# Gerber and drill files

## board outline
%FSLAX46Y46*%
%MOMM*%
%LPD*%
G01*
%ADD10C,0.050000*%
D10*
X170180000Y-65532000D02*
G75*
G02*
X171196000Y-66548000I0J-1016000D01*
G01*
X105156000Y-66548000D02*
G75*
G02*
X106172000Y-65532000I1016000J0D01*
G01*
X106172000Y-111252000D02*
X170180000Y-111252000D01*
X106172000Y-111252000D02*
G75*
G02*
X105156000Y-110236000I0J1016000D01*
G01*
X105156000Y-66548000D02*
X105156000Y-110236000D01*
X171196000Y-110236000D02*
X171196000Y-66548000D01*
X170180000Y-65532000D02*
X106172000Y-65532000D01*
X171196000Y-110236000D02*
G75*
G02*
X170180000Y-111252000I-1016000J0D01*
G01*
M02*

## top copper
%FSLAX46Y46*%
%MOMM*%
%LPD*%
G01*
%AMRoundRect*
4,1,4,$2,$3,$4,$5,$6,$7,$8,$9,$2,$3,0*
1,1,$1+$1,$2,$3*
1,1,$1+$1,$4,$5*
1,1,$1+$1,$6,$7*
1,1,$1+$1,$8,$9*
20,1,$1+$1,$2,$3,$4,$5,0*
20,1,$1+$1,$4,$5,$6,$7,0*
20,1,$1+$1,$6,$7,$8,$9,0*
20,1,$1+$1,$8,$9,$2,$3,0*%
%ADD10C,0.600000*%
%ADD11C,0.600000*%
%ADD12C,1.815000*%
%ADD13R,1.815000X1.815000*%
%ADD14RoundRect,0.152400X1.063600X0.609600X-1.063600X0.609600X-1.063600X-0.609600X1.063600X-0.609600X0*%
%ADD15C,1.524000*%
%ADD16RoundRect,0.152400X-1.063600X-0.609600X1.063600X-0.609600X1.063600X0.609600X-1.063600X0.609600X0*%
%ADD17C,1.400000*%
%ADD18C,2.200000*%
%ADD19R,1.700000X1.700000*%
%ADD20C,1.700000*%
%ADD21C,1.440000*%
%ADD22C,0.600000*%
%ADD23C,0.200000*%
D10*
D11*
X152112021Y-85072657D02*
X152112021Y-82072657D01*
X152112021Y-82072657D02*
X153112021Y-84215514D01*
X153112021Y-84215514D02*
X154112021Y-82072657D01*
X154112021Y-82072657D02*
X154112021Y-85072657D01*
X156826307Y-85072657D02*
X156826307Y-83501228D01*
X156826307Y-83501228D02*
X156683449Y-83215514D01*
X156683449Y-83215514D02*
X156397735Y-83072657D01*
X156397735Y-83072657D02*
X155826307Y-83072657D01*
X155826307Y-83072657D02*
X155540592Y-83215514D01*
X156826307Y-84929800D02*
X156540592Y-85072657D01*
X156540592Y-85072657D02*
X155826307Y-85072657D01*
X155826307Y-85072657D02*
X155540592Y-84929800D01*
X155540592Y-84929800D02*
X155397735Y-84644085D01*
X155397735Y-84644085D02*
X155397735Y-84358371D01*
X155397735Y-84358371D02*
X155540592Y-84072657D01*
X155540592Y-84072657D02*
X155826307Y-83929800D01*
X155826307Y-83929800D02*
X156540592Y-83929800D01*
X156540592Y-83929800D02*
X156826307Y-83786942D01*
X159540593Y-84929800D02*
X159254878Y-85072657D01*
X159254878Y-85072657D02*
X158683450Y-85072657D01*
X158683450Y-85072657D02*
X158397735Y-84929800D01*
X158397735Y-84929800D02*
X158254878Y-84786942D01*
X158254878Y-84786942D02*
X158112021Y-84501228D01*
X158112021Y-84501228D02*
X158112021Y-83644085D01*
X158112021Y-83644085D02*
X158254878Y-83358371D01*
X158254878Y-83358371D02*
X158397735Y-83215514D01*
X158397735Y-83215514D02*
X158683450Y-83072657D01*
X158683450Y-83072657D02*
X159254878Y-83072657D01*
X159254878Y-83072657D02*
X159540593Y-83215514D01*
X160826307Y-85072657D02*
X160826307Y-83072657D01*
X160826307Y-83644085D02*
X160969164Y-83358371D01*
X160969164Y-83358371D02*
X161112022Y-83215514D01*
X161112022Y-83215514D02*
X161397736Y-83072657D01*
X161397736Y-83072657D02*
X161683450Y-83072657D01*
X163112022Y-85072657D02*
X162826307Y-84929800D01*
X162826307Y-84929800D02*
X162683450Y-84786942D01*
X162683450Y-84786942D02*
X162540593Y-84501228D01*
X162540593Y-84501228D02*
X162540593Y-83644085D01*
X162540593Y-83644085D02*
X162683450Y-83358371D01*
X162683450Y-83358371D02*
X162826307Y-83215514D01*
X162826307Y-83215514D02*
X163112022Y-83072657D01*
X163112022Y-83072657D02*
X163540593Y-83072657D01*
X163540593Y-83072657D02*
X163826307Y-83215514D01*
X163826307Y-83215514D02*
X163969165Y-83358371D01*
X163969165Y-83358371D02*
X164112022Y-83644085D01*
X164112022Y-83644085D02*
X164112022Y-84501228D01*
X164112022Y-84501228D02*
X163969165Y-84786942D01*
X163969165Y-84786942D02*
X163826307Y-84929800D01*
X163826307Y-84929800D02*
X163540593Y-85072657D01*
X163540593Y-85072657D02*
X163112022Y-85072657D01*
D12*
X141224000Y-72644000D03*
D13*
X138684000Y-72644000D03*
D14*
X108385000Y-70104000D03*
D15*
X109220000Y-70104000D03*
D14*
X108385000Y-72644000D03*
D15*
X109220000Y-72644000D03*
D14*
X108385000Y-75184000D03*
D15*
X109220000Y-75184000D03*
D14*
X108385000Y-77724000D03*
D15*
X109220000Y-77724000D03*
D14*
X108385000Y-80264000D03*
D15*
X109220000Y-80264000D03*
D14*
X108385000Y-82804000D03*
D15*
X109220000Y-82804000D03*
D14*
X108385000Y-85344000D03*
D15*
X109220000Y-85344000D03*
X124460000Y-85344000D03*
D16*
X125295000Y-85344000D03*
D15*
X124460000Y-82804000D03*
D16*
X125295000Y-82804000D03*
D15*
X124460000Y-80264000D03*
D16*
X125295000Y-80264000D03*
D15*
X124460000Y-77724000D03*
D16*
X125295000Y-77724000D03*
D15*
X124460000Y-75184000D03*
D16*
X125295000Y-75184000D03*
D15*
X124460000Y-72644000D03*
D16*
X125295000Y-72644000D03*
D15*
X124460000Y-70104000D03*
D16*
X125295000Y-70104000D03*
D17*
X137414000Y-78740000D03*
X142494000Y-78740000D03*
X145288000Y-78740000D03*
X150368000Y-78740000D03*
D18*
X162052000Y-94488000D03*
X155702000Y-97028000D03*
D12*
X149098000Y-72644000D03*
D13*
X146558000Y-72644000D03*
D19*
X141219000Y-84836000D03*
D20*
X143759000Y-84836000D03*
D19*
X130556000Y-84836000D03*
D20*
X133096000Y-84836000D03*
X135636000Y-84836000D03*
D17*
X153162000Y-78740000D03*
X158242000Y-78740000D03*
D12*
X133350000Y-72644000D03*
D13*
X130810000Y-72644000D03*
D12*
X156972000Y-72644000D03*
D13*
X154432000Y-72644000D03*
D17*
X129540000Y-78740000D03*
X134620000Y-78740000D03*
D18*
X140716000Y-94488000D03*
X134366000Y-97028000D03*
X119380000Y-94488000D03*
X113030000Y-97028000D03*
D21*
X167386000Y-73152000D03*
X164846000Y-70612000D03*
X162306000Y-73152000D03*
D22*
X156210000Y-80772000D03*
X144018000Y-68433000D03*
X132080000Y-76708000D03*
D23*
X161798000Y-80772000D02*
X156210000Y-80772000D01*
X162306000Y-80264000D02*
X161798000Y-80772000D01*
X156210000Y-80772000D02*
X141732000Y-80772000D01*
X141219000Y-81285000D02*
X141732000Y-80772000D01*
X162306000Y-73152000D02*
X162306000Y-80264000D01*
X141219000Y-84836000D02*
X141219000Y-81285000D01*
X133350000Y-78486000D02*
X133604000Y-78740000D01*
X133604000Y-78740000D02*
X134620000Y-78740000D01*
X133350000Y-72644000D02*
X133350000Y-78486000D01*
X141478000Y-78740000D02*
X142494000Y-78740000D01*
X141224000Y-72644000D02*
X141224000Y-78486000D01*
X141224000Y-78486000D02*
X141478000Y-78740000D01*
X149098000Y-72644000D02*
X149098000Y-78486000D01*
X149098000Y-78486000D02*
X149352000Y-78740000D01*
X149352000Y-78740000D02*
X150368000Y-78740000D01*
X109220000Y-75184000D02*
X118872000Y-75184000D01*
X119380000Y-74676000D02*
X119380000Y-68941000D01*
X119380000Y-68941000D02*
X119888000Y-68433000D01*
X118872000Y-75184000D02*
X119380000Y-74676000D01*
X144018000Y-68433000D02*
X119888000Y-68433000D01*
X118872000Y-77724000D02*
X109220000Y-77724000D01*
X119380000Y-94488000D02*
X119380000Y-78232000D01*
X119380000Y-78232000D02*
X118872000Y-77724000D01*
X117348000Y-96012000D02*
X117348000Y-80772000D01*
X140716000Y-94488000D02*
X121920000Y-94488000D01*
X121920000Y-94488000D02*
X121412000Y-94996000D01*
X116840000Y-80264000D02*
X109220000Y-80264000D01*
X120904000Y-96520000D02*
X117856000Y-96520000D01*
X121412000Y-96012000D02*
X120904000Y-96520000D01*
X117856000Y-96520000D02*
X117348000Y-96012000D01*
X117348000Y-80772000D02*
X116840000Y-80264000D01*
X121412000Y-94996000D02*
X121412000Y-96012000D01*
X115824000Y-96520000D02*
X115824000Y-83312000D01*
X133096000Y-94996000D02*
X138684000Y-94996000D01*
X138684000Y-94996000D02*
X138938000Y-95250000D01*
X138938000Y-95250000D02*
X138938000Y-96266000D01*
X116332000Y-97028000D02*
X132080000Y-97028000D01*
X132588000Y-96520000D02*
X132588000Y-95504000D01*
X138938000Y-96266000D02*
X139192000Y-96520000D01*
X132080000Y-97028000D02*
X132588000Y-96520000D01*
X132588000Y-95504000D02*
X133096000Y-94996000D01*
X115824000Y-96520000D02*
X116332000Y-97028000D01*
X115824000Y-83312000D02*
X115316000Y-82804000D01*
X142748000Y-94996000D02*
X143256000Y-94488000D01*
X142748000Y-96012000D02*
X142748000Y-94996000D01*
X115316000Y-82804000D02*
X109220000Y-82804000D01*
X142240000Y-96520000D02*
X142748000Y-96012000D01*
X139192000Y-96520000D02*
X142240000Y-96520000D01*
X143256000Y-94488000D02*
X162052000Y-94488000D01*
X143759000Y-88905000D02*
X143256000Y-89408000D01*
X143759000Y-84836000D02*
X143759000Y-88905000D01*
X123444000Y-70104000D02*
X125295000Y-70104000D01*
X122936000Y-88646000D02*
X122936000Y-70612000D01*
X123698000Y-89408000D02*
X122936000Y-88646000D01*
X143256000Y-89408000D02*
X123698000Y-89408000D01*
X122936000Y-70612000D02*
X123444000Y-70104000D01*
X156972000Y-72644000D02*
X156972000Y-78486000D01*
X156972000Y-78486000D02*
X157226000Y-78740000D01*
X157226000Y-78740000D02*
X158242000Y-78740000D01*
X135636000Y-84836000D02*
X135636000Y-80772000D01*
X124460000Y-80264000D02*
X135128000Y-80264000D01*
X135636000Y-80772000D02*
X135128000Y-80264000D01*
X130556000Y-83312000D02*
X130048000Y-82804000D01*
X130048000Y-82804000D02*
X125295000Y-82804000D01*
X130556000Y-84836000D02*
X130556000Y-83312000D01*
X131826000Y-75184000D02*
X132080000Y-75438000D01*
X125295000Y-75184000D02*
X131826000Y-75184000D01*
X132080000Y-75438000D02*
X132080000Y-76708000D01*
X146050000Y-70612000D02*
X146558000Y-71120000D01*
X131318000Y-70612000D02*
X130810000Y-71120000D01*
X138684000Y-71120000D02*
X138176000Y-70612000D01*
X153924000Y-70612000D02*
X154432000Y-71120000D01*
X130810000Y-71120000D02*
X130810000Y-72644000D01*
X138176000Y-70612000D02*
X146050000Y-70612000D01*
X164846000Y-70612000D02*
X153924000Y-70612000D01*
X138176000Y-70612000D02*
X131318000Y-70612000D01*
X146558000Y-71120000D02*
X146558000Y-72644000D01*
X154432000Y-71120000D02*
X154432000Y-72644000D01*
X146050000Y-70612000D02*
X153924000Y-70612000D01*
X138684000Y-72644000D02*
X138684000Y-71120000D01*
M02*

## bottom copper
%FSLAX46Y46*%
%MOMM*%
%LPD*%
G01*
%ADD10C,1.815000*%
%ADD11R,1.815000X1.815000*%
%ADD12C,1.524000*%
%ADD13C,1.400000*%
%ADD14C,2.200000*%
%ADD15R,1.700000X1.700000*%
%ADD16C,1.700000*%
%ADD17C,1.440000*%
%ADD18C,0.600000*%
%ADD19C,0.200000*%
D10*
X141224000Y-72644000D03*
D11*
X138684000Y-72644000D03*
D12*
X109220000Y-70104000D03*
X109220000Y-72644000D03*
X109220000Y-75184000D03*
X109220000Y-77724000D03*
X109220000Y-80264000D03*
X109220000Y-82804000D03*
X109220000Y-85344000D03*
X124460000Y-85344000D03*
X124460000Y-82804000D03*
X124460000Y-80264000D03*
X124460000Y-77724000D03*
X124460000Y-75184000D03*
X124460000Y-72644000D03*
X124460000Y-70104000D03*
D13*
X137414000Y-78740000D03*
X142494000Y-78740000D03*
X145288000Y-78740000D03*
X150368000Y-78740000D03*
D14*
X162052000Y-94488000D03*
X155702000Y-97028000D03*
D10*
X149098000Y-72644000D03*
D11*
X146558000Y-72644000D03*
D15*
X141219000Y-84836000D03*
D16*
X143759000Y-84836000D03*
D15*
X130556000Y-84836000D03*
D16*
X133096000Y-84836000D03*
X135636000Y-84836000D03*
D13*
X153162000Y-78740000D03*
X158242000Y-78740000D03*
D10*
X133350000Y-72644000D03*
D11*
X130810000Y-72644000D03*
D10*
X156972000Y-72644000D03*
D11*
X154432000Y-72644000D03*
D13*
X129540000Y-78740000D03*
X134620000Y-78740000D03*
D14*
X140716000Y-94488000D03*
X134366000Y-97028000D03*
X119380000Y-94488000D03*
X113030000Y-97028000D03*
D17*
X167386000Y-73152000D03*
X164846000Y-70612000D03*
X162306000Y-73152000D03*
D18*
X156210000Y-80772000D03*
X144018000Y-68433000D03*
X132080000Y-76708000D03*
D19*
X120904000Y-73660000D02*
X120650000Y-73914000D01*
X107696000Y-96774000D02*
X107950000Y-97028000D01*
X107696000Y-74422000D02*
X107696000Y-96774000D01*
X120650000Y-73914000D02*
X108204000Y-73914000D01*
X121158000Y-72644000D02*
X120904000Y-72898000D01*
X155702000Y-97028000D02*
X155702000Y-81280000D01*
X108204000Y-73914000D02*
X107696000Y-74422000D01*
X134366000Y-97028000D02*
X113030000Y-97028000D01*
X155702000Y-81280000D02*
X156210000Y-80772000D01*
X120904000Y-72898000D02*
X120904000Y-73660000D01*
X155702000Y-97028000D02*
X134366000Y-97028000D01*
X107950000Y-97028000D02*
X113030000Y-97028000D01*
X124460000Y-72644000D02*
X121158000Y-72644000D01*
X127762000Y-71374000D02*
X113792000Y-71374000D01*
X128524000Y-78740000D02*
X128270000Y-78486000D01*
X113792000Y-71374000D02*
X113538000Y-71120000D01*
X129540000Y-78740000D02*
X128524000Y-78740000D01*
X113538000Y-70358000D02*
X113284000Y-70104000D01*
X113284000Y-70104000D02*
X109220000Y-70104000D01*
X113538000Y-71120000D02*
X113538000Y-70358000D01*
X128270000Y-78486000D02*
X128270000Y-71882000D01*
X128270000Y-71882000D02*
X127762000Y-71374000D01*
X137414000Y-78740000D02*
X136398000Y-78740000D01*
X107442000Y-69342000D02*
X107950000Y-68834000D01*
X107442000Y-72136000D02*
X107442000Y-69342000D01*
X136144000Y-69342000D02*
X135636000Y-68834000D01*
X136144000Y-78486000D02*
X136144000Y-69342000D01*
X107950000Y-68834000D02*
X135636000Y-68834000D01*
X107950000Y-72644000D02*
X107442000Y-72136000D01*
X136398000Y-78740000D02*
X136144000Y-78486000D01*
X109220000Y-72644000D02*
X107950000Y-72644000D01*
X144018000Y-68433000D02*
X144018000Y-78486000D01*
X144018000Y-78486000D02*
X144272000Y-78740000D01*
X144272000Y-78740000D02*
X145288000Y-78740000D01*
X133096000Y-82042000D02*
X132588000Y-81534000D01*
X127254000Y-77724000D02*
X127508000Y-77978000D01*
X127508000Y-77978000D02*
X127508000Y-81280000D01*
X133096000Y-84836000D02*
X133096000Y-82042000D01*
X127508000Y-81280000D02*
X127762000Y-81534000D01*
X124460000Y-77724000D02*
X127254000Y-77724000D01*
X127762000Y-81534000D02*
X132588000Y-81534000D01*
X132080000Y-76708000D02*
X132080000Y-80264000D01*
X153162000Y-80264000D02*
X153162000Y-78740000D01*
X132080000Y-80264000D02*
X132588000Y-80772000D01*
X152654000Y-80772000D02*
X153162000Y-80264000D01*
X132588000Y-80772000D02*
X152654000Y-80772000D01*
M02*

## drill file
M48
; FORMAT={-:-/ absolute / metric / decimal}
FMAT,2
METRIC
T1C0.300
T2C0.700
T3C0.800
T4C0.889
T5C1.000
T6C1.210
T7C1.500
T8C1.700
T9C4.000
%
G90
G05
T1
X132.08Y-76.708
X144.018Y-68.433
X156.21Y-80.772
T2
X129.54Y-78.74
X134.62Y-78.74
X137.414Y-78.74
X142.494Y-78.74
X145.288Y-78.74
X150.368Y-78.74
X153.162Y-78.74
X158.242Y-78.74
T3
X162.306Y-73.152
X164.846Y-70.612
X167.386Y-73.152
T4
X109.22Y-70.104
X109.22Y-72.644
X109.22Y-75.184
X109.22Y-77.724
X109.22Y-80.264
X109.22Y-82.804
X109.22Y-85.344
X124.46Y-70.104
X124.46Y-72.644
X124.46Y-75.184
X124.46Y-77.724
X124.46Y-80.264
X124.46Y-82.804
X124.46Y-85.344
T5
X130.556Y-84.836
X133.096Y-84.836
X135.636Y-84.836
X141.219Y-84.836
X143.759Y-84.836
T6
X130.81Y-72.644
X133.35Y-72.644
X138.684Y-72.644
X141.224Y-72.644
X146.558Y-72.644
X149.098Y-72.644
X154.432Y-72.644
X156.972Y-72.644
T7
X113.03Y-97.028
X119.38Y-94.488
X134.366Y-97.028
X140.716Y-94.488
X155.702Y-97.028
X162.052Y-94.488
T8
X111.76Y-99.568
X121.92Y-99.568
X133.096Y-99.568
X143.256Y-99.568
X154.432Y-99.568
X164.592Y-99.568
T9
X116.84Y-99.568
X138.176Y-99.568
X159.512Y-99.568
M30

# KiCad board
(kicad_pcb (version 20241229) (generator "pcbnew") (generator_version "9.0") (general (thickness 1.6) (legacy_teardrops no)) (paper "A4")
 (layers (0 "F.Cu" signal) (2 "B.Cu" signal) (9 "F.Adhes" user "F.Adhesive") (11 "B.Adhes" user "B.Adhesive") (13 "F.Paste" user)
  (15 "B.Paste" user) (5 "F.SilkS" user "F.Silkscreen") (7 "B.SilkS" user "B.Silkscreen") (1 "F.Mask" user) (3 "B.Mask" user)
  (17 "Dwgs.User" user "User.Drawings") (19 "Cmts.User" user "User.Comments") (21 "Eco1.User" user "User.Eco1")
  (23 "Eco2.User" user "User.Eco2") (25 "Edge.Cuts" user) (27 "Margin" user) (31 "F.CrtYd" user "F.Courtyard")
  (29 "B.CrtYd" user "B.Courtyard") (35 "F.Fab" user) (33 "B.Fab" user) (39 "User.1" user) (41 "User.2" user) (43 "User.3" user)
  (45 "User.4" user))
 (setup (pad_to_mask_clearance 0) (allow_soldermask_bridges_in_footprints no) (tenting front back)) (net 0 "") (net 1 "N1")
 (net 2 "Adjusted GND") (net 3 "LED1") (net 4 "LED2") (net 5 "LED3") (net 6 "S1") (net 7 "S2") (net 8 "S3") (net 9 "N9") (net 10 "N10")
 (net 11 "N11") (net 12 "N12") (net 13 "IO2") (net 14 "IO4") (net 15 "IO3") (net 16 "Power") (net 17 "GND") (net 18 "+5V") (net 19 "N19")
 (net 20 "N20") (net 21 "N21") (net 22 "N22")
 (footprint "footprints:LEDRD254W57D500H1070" (layer "F.Cu") (at 139.954 72.644)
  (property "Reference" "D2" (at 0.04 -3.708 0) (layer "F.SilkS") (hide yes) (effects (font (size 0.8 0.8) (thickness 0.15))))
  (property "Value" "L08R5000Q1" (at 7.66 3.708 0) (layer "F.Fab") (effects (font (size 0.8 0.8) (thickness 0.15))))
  (pad "A" thru_hole circle (at 1.27 0) (size 1.815 1.815) (drill 1.21) (layers "*.Cu" "*.Mask") (remove_unused_layers no) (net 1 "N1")
   (solder_mask_margin 0.102))
  (pad "C" thru_hole rect (at -1.27 0) (size 1.815 1.815) (drill 1.21) (layers "*.Cu" "*.Mask") (remove_unused_layers no)
   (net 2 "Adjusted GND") (solder_mask_margin 0.102)))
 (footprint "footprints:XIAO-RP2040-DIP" (layer "F.Cu") (at 116.84 77.724)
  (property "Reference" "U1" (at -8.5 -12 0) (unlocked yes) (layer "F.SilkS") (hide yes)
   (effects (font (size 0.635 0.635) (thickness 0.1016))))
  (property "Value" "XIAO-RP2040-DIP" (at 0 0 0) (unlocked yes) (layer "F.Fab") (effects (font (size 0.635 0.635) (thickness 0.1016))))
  (pad "1" smd roundrect (at -8.455 -7.62 180) (size 2.432 1.524) (layers "F.Cu" "F.Mask") (roundrect_rratio 0.1) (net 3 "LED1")
   (thermal_bridge_angle 45))
  (pad "1" thru_hole circle (at -7.62 -7.62 180) (size 1.524 1.524) (drill 0.889) (layers "*.Cu" "*.Mask") (remove_unused_layers no)
   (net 3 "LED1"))
  (pad "2" smd roundrect (at -8.455 -5.08 180) (size 2.432 1.524) (layers "F.Cu" "F.Mask") (roundrect_rratio 0.1) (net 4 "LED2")
   (thermal_bridge_angle 45))
  (pad "2" thru_hole circle (at -7.62 -5.08 180) (size 1.524 1.524) (drill 0.889) (layers "*.Cu" "*.Mask") (remove_unused_layers no)
   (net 4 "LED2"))
  (pad "3" smd roundrect (at -8.455 -2.54 180) (size 2.432 1.524) (layers "F.Cu" "F.Mask") (roundrect_rratio 0.1) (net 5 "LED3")
   (thermal_bridge_angle 45))
  (pad "3" thru_hole circle (at -7.62 -2.54 180) (size 1.524 1.524) (drill 0.889) (layers "*.Cu" "*.Mask") (remove_unused_layers no)
   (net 5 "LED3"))
  (pad "4" smd roundrect (at -8.455 0 180) (size 2.432 1.524) (layers "F.Cu" "F.Mask") (roundrect_rratio 0.1) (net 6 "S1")
   (thermal_bridge_angle 45))
  (pad "4" thru_hole circle (at -7.62 0 180) (size 1.524 1.524) (drill 0.889) (layers "*.Cu" "*.Mask") (remove_unused_layers no)
   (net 6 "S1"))
  (pad "5" smd roundrect (at -8.455 2.54 180) (size 2.432 1.524) (layers "F.Cu" "F.Mask") (roundrect_rratio 0.1) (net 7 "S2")
   (thermal_bridge_angle 45))
  (pad "5" thru_hole circle (at -7.62 2.54 180) (size 1.524 1.524) (drill 0.889) (layers "*.Cu" "*.Mask") (remove_unused_layers no)
   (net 7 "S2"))
  (pad "6" smd roundrect (at -8.455 5.08 180) (size 2.432 1.524) (layers "F.Cu" "F.Mask") (roundrect_rratio 0.1) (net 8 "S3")
   (thermal_bridge_angle 45))
  (pad "6" thru_hole circle (at -7.62 5.08 180) (size 1.524 1.524) (drill 0.889) (layers "*.Cu" "*.Mask") (remove_unused_layers no)
   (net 8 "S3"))
  (pad "7" smd roundrect (at -8.455 7.62 180) (size 2.432 1.524) (layers "F.Cu" "F.Mask") (roundrect_rratio 0.1) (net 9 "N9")
   (thermal_bridge_angle 45))
  (pad "7" thru_hole circle (at -7.62 7.62 180) (size 1.524 1.524) (drill 0.889) (layers "*.Cu" "*.Mask") (remove_unused_layers no)
   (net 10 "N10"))
  (pad "8" thru_hole circle (at 7.62 7.62) (size 1.524 1.524) (drill 0.889) (layers "*.Cu" "*.Mask") (remove_unused_layers no)
   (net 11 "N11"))
  (pad "8" smd roundrect (at 8.455 7.62) (size 2.432 1.524) (layers "F.Cu" "F.Mask") (roundrect_rratio 0.1) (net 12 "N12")
   (thermal_bridge_angle 45))
  (pad "9" thru_hole circle (at 7.62 5.08) (size 1.524 1.524) (drill 0.889) (layers "*.Cu" "*.Mask") (remove_unused_layers no)
   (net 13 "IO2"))
  (pad "9" smd roundrect (at 8.455 5.08) (size 2.432 1.524) (layers "F.Cu" "F.Mask") (roundrect_rratio 0.1) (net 13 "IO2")
   (thermal_bridge_angle 45))
  (pad "10" thru_hole circle (at 7.62 2.54) (size 1.524 1.524) (drill 0.889) (layers "*.Cu" "*.Mask") (remove_unused_layers no)
   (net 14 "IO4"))
  (pad "10" smd roundrect (at 8.455 2.54) (size 2.432 1.524) (layers "F.Cu" "F.Mask") (roundrect_rratio 0.1) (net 14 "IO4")
   (thermal_bridge_angle 45))
  (pad "11" thru_hole circle (at 7.62 0) (size 1.524 1.524) (drill 0.889) (layers "*.Cu" "*.Mask") (remove_unused_layers no) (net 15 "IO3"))
  (pad "11" smd roundrect (at 8.455 0) (size 2.432 1.524) (layers "F.Cu" "F.Mask") (roundrect_rratio 0.1) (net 15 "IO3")
   (thermal_bridge_angle 45))
  (pad "12" thru_hole circle (at 7.62 -2.54) (size 1.524 1.524) (drill 0.889) (layers "*.Cu" "*.Mask") (remove_unused_layers no)
   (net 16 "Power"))
  (pad "12" smd roundrect (at 8.455 -2.54) (size 2.432 1.524) (layers "F.Cu" "F.Mask") (roundrect_rratio 0.1) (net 16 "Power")
   (thermal_bridge_angle 45))
  (pad "13" thru_hole circle (at 7.62 -5.08) (size 1.524 1.524) (drill 0.889) (layers "*.Cu" "*.Mask") (remove_unused_layers no)
   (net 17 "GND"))
  (pad "13" smd roundrect (at 8.455 -5.08) (size 2.432 1.524) (layers "F.Cu" "F.Mask") (roundrect_rratio 0.1) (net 17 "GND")
   (thermal_bridge_angle 45))
  (pad "14" thru_hole circle (at 7.62 -7.62) (size 1.524 1.524) (drill 0.889) (layers "*.Cu" "*.Mask") (remove_unused_layers no)
   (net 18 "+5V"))
  (pad "14" smd roundrect (at 8.455 -7.62) (size 2.432 1.524) (layers "F.Cu" "F.Mask") (roundrect_rratio 0.1) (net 18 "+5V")
   (thermal_bridge_angle 45)))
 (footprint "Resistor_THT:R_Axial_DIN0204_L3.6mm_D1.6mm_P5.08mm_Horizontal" (layer "F.Cu") (at 137.414 78.74)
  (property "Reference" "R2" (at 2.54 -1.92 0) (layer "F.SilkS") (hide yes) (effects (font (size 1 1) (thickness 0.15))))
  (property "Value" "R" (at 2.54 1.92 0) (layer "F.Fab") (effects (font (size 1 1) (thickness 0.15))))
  (pad "1" thru_hole circle (at 0 0) (size 1.4 1.4) (drill 0.7) (layers "*.Cu" "*.Mask") (remove_unused_layers no) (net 4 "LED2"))
  (pad "2" thru_hole circle (at 5.08 0) (size 1.4 1.4) (drill 0.7) (layers "*.Cu" "*.Mask") (remove_unused_layers no) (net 1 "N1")))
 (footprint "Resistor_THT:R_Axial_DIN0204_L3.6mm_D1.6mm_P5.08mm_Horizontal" (layer "F.Cu") (at 145.288 78.74)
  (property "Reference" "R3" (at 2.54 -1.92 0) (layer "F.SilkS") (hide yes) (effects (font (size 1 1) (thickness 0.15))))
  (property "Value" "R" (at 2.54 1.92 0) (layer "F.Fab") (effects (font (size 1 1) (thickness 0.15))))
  (pad "1" thru_hole circle (at 0 0) (size 1.4 1.4) (drill 0.7) (layers "*.Cu" "*.Mask") (remove_unused_layers no) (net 5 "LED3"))
  (pad "2" thru_hole circle (at 5.08 0) (size 1.4 1.4) (drill 0.7) (layers "*.Cu" "*.Mask") (remove_unused_layers no) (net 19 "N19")))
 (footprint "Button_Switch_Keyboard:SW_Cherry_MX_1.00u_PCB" (layer "F.Cu") (at 162.052 94.488)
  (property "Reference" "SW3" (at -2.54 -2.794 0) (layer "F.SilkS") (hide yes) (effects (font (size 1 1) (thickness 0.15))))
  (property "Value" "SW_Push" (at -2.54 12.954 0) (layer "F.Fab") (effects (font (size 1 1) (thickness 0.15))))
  (pad "" np_thru_hole circle (at -7.62 5.08) (size 1.7 1.7) (drill 1.7) (layers "*.Cu" "*.Mask"))
  (pad "" np_thru_hole circle (at -2.54 5.08) (size 4 4) (drill 4) (layers "*.Cu" "*.Mask"))
  (pad "" np_thru_hole circle (at 2.54 5.08) (size 1.7 1.7) (drill 1.7) (layers "*.Cu" "*.Mask"))
  (pad "1" thru_hole circle (at 0 0) (size 2.2 2.2) (drill 1.5) (layers "*.Cu" "*.Mask") (remove_unused_layers no) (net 8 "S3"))
  (pad "2" thru_hole circle (at -6.35 2.54) (size 2.2 2.2) (drill 1.5) (layers "*.Cu" "*.Mask") (remove_unused_layers no) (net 17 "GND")))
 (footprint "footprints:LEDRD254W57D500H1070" (layer "F.Cu") (at 147.828 72.644)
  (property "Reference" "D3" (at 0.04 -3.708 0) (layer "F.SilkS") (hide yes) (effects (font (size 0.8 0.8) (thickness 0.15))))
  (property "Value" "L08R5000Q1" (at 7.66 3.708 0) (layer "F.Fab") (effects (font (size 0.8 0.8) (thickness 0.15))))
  (pad "A" thru_hole circle (at 1.27 0) (size 1.815 1.815) (drill 1.21) (layers "*.Cu" "*.Mask") (remove_unused_layers no) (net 19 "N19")
   (solder_mask_margin 0.102))
  (pad "C" thru_hole rect (at -1.27 0) (size 1.815 1.815) (drill 1.21) (layers "*.Cu" "*.Mask") (remove_unused_layers no)
   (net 2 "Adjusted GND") (solder_mask_margin 0.102)))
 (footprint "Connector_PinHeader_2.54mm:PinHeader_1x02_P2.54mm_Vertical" (layer "F.Cu") (at 141.219 84.836 90)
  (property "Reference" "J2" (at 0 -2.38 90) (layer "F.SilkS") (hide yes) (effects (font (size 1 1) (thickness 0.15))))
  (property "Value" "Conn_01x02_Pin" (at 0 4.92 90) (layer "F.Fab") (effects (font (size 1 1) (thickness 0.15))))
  (pad "1" thru_hole rect (at 0 0 90) (size 1.7 1.7) (drill 1) (layers "*.Cu" "*.Mask") (remove_unused_layers no) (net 17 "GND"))
  (pad "2" thru_hole circle (at 0 2.54 90) (size 1.7 1.7) (drill 1) (layers "*.Cu" "*.Mask") (remove_unused_layers no) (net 18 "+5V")))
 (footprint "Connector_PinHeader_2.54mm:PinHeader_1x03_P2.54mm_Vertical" (layer "F.Cu") (at 130.556 84.836 90)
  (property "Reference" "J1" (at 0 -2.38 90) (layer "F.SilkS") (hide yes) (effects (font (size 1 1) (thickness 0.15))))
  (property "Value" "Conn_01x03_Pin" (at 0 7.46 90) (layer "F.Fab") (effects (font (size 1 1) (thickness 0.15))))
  (pad "1" thru_hole rect (at 0 0 90) (size 1.7 1.7) (drill 1) (layers "*.Cu" "*.Mask") (remove_unused_layers no) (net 13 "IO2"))
  (pad "2" thru_hole circle (at 0 2.54 90) (size 1.7 1.7) (drill 1) (layers "*.Cu" "*.Mask") (remove_unused_layers no) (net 15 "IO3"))
  (pad "3" thru_hole circle (at 0 5.08 90) (size 1.7 1.7) (drill 1) (layers "*.Cu" "*.Mask") (remove_unused_layers no) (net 14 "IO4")))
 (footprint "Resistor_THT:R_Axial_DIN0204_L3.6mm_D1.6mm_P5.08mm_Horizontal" (layer "F.Cu") (at 153.162 78.74)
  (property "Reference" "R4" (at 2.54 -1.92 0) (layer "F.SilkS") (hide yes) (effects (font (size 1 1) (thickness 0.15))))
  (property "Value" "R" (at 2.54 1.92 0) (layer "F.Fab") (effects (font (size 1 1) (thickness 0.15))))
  (pad "1" thru_hole circle (at 0 0) (size 1.4 1.4) (drill 0.7) (layers "*.Cu" "*.Mask") (remove_unused_layers no) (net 16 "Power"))
  (pad "2" thru_hole circle (at 5.08 0) (size 1.4 1.4) (drill 0.7) (layers "*.Cu" "*.Mask") (remove_unused_layers no) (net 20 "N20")))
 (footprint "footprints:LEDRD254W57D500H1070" (layer "F.Cu") (at 132.08 72.644)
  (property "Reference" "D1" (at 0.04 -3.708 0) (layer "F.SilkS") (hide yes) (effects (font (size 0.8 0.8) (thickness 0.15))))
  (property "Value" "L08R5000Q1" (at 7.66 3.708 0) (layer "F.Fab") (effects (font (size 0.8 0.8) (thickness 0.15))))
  (pad "A" thru_hole circle (at 1.27 0) (size 1.815 1.815) (drill 1.21) (layers "*.Cu" "*.Mask") (remove_unused_layers no) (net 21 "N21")
   (solder_mask_margin 0.102))
  (pad "C" thru_hole rect (at -1.27 0) (size 1.815 1.815) (drill 1.21) (layers "*.Cu" "*.Mask") (remove_unused_layers no)
   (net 2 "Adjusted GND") (solder_mask_margin 0.102)))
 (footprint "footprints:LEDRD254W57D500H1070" (layer "F.Cu") (at 155.702 72.644)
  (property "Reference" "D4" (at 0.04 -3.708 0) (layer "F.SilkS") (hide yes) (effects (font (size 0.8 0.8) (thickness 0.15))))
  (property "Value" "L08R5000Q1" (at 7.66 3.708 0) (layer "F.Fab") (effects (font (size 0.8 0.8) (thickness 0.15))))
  (pad "A" thru_hole circle (at 1.27 0) (size 1.815 1.815) (drill 1.21) (layers "*.Cu" "*.Mask") (remove_unused_layers no) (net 20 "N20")
   (solder_mask_margin 0.102))
  (pad "C" thru_hole rect (at -1.27 0) (size 1.815 1.815) (drill 1.21) (layers "*.Cu" "*.Mask") (remove_unused_layers no)
   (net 2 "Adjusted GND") (solder_mask_margin 0.102)))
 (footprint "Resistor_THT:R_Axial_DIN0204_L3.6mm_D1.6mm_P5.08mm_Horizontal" (layer "F.Cu") (at 129.54 78.74)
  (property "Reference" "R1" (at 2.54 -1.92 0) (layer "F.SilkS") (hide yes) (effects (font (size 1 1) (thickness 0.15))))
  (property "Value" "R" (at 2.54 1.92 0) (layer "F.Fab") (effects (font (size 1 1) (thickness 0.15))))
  (pad "1" thru_hole circle (at 0 0) (size 1.4 1.4) (drill 0.7) (layers "*.Cu" "*.Mask") (remove_unused_layers no) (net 3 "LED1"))
  (pad "2" thru_hole circle (at 5.08 0) (size 1.4 1.4) (drill 0.7) (layers "*.Cu" "*.Mask") (remove_unused_layers no) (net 21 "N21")))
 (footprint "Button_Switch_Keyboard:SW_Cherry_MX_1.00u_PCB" (layer "F.Cu") (at 140.716 94.488)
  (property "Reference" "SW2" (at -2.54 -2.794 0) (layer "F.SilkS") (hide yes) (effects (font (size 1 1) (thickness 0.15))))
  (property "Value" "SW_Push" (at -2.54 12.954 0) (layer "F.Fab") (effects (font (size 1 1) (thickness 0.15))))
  (pad "" np_thru_hole circle (at -7.62 5.08) (size 1.7 1.7) (drill 1.7) (layers "*.Cu" "*.Mask"))
  (pad "" np_thru_hole circle (at -2.54 5.08) (size 4 4) (drill 4) (layers "*.Cu" "*.Mask"))
  (pad "" np_thru_hole circle (at 2.54 5.08) (size 1.7 1.7) (drill 1.7) (layers "*.Cu" "*.Mask"))
  (pad "1" thru_hole circle (at 0 0) (size 2.2 2.2) (drill 1.5) (layers "*.Cu" "*.Mask") (remove_unused_layers no) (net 7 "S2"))
  (pad "2" thru_hole circle (at -6.35 2.54) (size 2.2 2.2) (drill 1.5) (layers "*.Cu" "*.Mask") (remove_unused_layers no) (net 17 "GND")))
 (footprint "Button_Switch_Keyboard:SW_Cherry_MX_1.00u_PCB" (layer "F.Cu") (at 119.38 94.488)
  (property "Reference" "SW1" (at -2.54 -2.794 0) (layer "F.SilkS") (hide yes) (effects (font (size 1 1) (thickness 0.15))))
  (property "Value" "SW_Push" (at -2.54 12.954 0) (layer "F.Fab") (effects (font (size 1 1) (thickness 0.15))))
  (pad "" np_thru_hole circle (at -7.62 5.08) (size 1.7 1.7) (drill 1.7) (layers "*.Cu" "*.Mask"))
  (pad "" np_thru_hole circle (at -2.54 5.08) (size 4 4) (drill 4) (layers "*.Cu" "*.Mask"))
  (pad "" np_thru_hole circle (at 2.54 5.08) (size 1.7 1.7) (drill 1.7) (layers "*.Cu" "*.Mask"))
  (pad "1" thru_hole circle (at 0 0) (size 2.2 2.2) (drill 1.5) (layers "*.Cu" "*.Mask") (remove_unused_layers no) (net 6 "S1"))
  (pad "2" thru_hole circle (at -6.35 2.54) (size 2.2 2.2) (drill 1.5) (layers "*.Cu" "*.Mask") (remove_unused_layers no) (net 17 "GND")))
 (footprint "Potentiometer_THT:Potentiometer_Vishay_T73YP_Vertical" (layer "F.Cu") (at 167.386 73.152 90)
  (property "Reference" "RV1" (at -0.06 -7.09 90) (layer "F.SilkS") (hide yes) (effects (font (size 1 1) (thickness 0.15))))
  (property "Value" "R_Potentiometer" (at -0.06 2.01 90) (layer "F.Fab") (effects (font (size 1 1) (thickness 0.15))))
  (pad "1" thru_hole circle (at 0 0 90) (size 1.44 1.44) (drill 0.8) (layers "*.Cu" "*.Mask") (remove_unused_layers no) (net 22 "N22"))
  (pad "2" thru_hole circle (at 2.54 -2.54 90) (size 1.44 1.44) (drill 0.8) (layers "*.Cu" "*.Mask") (remove_unused_layers no)
   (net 2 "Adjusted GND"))
  (pad "3" thru_hole circle (at 0 -5.08 90) (size 1.44 1.44) (drill 0.8) (layers "*.Cu" "*.Mask") (remove_unused_layers no) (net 17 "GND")))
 (gr_arc (start 170.18 65.532) (mid 170.89842 65.82958) (end 171.196 66.548) (stroke (width 0.05) (type default)) (layer "Edge.Cuts"))
 (gr_arc (start 105.156 66.548) (mid 105.45358 65.82958) (end 106.172 65.532) (stroke (width 0.05) (type default)) (layer "Edge.Cuts"))
 (gr_line (start 106.172 111.252) (end 170.18 111.252) (stroke (width 0.05) (type default)) (layer "Edge.Cuts"))
 (gr_arc (start 106.172 111.252) (mid 105.45358 110.95442) (end 105.156 110.236) (stroke (width 0.05) (type default)) (layer "Edge.Cuts"))
 (gr_line (start 105.156 66.548) (end 105.156 110.236) (stroke (width 0.05) (type default)) (layer "Edge.Cuts"))
 (gr_line (start 171.196 110.236) (end 171.196 66.548) (stroke (width 0.05) (type default)) (layer "Edge.Cuts"))
 (gr_line (start 170.18 65.532) (end 106.172 65.532) (stroke (width 0.05) (type default)) (layer "Edge.Cuts"))
 (gr_arc (start 171.196 110.236) (mid 170.89842 110.95442) (end 170.18 111.252) (stroke (width 0.05) (type default)) (layer "Edge.Cuts"))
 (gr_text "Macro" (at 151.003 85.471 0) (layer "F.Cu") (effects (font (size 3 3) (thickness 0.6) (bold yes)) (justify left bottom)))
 (segment (start 161.798 80.772) (end 156.21 80.772) (width 0.2) (layer "F.Cu") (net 17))
 (segment (start 162.306 80.264) (end 161.798 80.772) (width 0.2) (layer "F.Cu") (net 17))
 (segment (start 156.21 80.772) (end 141.732 80.772) (width 0.2) (layer "F.Cu") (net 17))
 (segment (start 141.219 81.285) (end 141.732 80.772) (width 0.2) (layer "F.Cu") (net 17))
 (segment (start 162.306 73.152) (end 162.306 80.264) (width 0.2) (layer "F.Cu") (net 17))
 (segment (start 141.219 84.836) (end 141.219 81.285) (width 0.2) (layer "F.Cu") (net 17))
 (via (at 156.21 80.772) (size 0.6) (drill 0.3) (layers "F.Cu" "B.Cu") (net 17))
 (segment (start 120.904 73.66) (end 120.65 73.914) (width 0.2) (layer "B.Cu") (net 17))
 (segment (start 107.696 96.774) (end 107.95 97.028) (width 0.2) (layer "B.Cu") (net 17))
 (segment (start 107.696 74.422) (end 107.696 96.774) (width 0.2) (layer "B.Cu") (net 17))
 (segment (start 120.65 73.914) (end 108.204 73.914) (width 0.2) (layer "B.Cu") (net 17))
 (segment (start 121.158 72.644) (end 120.904 72.898) (width 0.2) (layer "B.Cu") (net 17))
 (segment (start 155.702 97.028) (end 155.702 81.28) (width 0.2) (layer "B.Cu") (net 17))
 (segment (start 108.204 73.914) (end 107.696 74.422) (width 0.2) (layer "B.Cu") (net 17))
 (segment (start 134.366 97.028) (end 113.03 97.028) (width 0.2) (layer "B.Cu") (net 17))
 (segment (start 155.702 81.28) (end 156.21 80.772) (width 0.2) (layer "B.Cu") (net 17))
 (segment (start 120.904 72.898) (end 120.904 73.66) (width 0.2) (layer "B.Cu") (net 17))
 (segment (start 155.702 97.028) (end 134.366 97.028) (width 0.2) (layer "B.Cu") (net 17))
 (segment (start 107.95 97.028) (end 113.03 97.028) (width 0.2) (layer "B.Cu") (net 17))
 (segment (start 124.46 72.644) (end 121.158 72.644) (width 0.2) (layer "B.Cu") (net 17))
 (segment (start 133.35 78.486) (end 133.604 78.74) (width 0.2) (layer "F.Cu") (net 21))
 (segment (start 133.604 78.74) (end 134.62 78.74) (width 0.2) (layer "F.Cu") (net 21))
 (segment (start 133.35 72.644) (end 133.35 78.486) (width 0.2) (layer "F.Cu") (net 21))
 (segment (start 141.478 78.74) (end 142.494 78.74) (width 0.2) (layer "F.Cu") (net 1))
 (segment (start 141.224 72.644) (end 141.224 78.486) (width 0.2) (layer "F.Cu") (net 1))
 (segment (start 141.224 78.486) (end 141.478 78.74) (width 0.2) (layer "F.Cu") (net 1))
 (segment (start 149.098 72.644) (end 149.098 78.486) (width 0.2) (layer "F.Cu") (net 19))
 (segment (start 149.098 78.486) (end 149.352 78.74) (width 0.2) (layer "F.Cu") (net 19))
 (segment (start 149.352 78.74) (end 150.368 78.74) (width 0.2) (layer "F.Cu") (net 19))
 (segment (start 127.762 71.374) (end 113.792 71.374) (width 0.2) (layer "B.Cu") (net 3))
 (segment (start 128.524 78.74) (end 128.27 78.486) (width 0.2) (layer "B.Cu") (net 3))
 (segment (start 113.792 71.374) (end 113.538 71.12) (width 0.2) (layer "B.Cu") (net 3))
 (segment (start 129.54 78.74) (end 128.524 78.74) (width 0.2) (layer "B.Cu") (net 3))
 (segment (start 113.538 70.358) (end 113.284 70.104) (width 0.2) (layer "B.Cu") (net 3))
 (segment (start 113.284 70.104) (end 109.22 70.104) (width 0.2) (layer "B.Cu") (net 3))
 (segment (start 113.538 71.12) (end 113.538 70.358) (width 0.2) (layer "B.Cu") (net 3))
 (segment (start 128.27 78.486) (end 128.27 71.882) (width 0.2) (layer "B.Cu") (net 3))
 (segment (start 128.27 71.882) (end 127.762 71.374) (width 0.2) (layer "B.Cu") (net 3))
 (segment (start 137.414 78.74) (end 136.398 78.74) (width 0.2) (layer "B.Cu") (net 4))
 (segment (start 107.442 69.342) (end 107.95 68.834) (width 0.2) (layer "B.Cu") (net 4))
 (segment (start 107.442 72.136) (end 107.442 69.342) (width 0.2) (layer "B.Cu") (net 4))
 (segment (start 136.144 69.342) (end 135.636 68.834) (width 0.2) (layer "B.Cu") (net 4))
 (segment (start 136.144 78.486) (end 136.144 69.342) (width 0.2) (layer "B.Cu") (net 4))
 (segment (start 107.95 68.834) (end 135.636 68.834) (width 0.2) (layer "B.Cu") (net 4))
 (segment (start 107.95 72.644) (end 107.442 72.136) (width 0.2) (layer "B.Cu") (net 4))
 (segment (start 136.398 78.74) (end 136.144 78.486) (width 0.2) (layer "B.Cu") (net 4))
 (segment (start 109.22 72.644) (end 107.95 72.644) (width 0.2) (layer "B.Cu") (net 4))
 (segment (start 109.22 75.184) (end 118.872 75.184) (width 0.2) (layer "F.Cu") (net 5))
 (segment (start 119.38 74.676) (end 119.38 68.941) (width 0.2) (layer "F.Cu") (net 5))
 (segment (start 119.38 68.941) (end 119.888 68.433) (width 0.2) (layer "F.Cu") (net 5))
 (segment (start 118.872 75.184) (end 119.38 74.676) (width 0.2) (layer "F.Cu") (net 5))
 (segment (start 144.018 68.433) (end 119.888 68.433) (width 0.2) (layer "F.Cu") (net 5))
 (via (at 144.018 68.433) (size 0.6) (drill 0.3) (layers "F.Cu" "B.Cu") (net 5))
 (segment (start 144.018 68.433) (end 144.018 78.486) (width 0.2) (layer "B.Cu") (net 5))
 (segment (start 144.018 78.486) (end 144.272 78.74) (width 0.2) (layer "B.Cu") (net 5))
 (segment (start 144.272 78.74) (end 145.288 78.74) (width 0.2) (layer "B.Cu") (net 5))
 (segment (start 118.872 77.724) (end 109.22 77.724) (width 0.2) (layer "F.Cu") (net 6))
 (segment (start 119.38 94.488) (end 119.38 78.232) (width 0.2) (layer "F.Cu") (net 6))
 (segment (start 119.38 78.232) (end 118.872 77.724) (width 0.2) (layer "F.Cu") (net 6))
 (segment (start 117.348 96.012) (end 117.348 80.772) (width 0.2) (layer "F.Cu") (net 7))
 (segment (start 140.716 94.488) (end 121.92 94.488) (width 0.2) (layer "F.Cu") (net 7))
 (segment (start 121.92 94.488) (end 121.412 94.996) (width 0.2) (layer "F.Cu") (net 7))
 (segment (start 116.84 80.264) (end 109.22 80.264) (width 0.2) (layer "F.Cu") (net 7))
 (segment (start 120.904 96.52) (end 117.856 96.52) (width 0.2) (layer "F.Cu") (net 7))
 (segment (start 121.412 96.012) (end 120.904 96.52) (width 0.2) (layer "F.Cu") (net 7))
 (segment (start 117.856 96.52) (end 117.348 96.012) (width 0.2) (layer "F.Cu") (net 7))
 (segment (start 117.348 80.772) (end 116.84 80.264) (width 0.2) (layer "F.Cu") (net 7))
 (segment (start 121.412 94.996) (end 121.412 96.012) (width 0.2) (layer "F.Cu") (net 7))
 (segment (start 115.824 96.52) (end 115.824 83.312) (width 0.2) (layer "F.Cu") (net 8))
 (segment (start 133.096 94.996) (end 138.684 94.996) (width 0.2) (layer "F.Cu") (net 8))
 (segment (start 138.684 94.996) (end 138.938 95.25) (width 0.2) (layer "F.Cu") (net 8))
 (segment (start 138.938 95.25) (end 138.938 96.266) (width 0.2) (layer "F.Cu") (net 8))
 (segment (start 116.332 97.028) (end 132.08 97.028) (width 0.2) (layer "F.Cu") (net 8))
 (segment (start 132.588 96.52) (end 132.588 95.504) (width 0.2) (layer "F.Cu") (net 8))
 (segment (start 138.938 96.266) (end 139.192 96.52) (width 0.2) (layer "F.Cu") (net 8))
 (segment (start 132.08 97.028) (end 132.588 96.52) (width 0.2) (layer "F.Cu") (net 8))
 (segment (start 132.588 95.504) (end 133.096 94.996) (width 0.2) (layer "F.Cu") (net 8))
 (segment (start 115.824 96.52) (end 116.332 97.028) (width 0.2) (layer "F.Cu") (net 8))
 (segment (start 115.824 83.312) (end 115.316 82.804) (width 0.2) (layer "F.Cu") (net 8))
 (segment (start 142.748 94.996) (end 143.256 94.488) (width 0.2) (layer "F.Cu") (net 8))
 (segment (start 142.748 96.012) (end 142.748 94.996) (width 0.2) (layer "F.Cu") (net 8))
 (segment (start 115.316 82.804) (end 109.22 82.804) (width 0.2) (layer "F.Cu") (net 8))
 (segment (start 142.24 96.52) (end 142.748 96.012) (width 0.2) (layer "F.Cu") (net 8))
 (segment (start 139.192 96.52) (end 142.24 96.52) (width 0.2) (layer "F.Cu") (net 8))
 (segment (start 143.256 94.488) (end 162.052 94.488) (width 0.2) (layer "F.Cu") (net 8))
 (segment (start 143.759 88.905) (end 143.256 89.408) (width 0.2) (layer "F.Cu") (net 18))
 (segment (start 143.759 84.836) (end 143.759 88.905) (width 0.2) (layer "F.Cu") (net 18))
 (segment (start 123.444 70.104) (end 125.295 70.104) (width 0.2) (layer "F.Cu") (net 18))
 (segment (start 122.936 88.646) (end 122.936 70.612) (width 0.2) (layer "F.Cu") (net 18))
 (segment (start 123.698 89.408) (end 122.936 88.646) (width 0.2) (layer "F.Cu") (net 18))
 (segment (start 143.256 89.408) (end 123.698 89.408) (width 0.2) (layer "F.Cu") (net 18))
 (segment (start 122.936 70.612) (end 123.444 70.104) (width 0.2) (layer "F.Cu") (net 18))
 (segment (start 156.972 72.644) (end 156.972 78.486) (width 0.2) (layer "F.Cu") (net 20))
 (segment (start 156.972 78.486) (end 157.226 78.74) (width 0.2) (layer "F.Cu") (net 20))
 (segment (start 157.226 78.74) (end 158.242 78.74) (width 0.2) (layer "F.Cu") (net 20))
 (segment (start 133.096 82.042) (end 132.588 81.534) (width 0.2) (layer "B.Cu") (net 15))
 (segment (start 127.254 77.724) (end 127.508 77.978) (width 0.2) (layer "B.Cu") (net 15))
 (segment (start 127.508 77.978) (end 127.508 81.28) (width 0.2) (layer "B.Cu") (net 15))
 (segment (start 133.096 84.836) (end 133.096 82.042) (width 0.2) (layer "B.Cu") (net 15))
 (segment (start 127.508 81.28) (end 127.762 81.534) (width 0.2) (layer "B.Cu") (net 15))
 (segment (start 124.46 77.724) (end 127.254 77.724) (width 0.2) (layer "B.Cu") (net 15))
 (segment (start 127.762 81.534) (end 132.588 81.534) (width 0.2) (layer "B.Cu") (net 15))
 (segment (start 135.636 84.836) (end 135.636 80.772) (width 0.2) (layer "F.Cu") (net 14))
 (segment (start 124.46 80.264) (end 135.128 80.264) (width 0.2) (layer "F.Cu") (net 14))
 (segment (start 135.636 80.772) (end 135.128 80.264) (width 0.2) (layer "F.Cu") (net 14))
 (segment (start 130.556 83.312) (end 130.048 82.804) (width 0.2) (layer "F.Cu") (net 13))
 (segment (start 130.048 82.804) (end 125.295 82.804) (width 0.2) (layer "F.Cu") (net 13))
 (segment (start 130.556 84.836) (end 130.556 83.312) (width 0.2) (layer "F.Cu") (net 13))
 (segment (start 131.826 75.184) (end 132.08 75.438) (width 0.2) (layer "F.Cu") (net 16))
 (segment (start 125.295 75.184) (end 131.826 75.184) (width 0.2) (layer "F.Cu") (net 16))
 (segment (start 132.08 75.438) (end 132.08 76.708) (width 0.2) (layer "F.Cu") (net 16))
 (via (at 132.08 76.708) (size 0.6) (drill 0.3) (layers "F.Cu" "B.Cu") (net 16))
 (segment (start 132.08 76.708) (end 132.08 80.264) (width 0.2) (layer "B.Cu") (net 16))
 (segment (start 153.162 80.264) (end 153.162 78.74) (width 0.2) (layer "B.Cu") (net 16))
 (segment (start 132.08 80.264) (end 132.588 80.772) (width 0.2) (layer "B.Cu") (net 16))
 (segment (start 152.654 80.772) (end 153.162 80.264) (width 0.2) (layer "B.Cu") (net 16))
 (segment (start 132.588 80.772) (end 152.654 80.772) (width 0.2) (layer "B.Cu") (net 16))
 (segment (start 146.05 70.612) (end 146.558 71.12) (width 0.2) (layer "F.Cu") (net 2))
 (segment (start 131.318 70.612) (end 130.81 71.12) (width 0.2) (layer "F.Cu") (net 2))
 (segment (start 138.684 71.12) (end 138.176 70.612) (width 0.2) (layer "F.Cu") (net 2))
 (segment (start 153.924 70.612) (end 154.432 71.12) (width 0.2) (layer "F.Cu") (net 2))
 (segment (start 130.81 71.12) (end 130.81 72.644) (width 0.2) (layer "F.Cu") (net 2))
 (segment (start 138.176 70.612) (end 146.05 70.612) (width 0.2) (layer "F.Cu") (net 2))
 (segment (start 164.846 70.612) (end 153.924 70.612) (width 0.2) (layer "F.Cu") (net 2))
 (segment (start 138.176 70.612) (end 131.318 70.612) (width 0.2) (layer "F.Cu") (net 2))
 (segment (start 146.558 71.12) (end 146.558 72.644) (width 0.2) (layer "F.Cu") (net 2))
 (segment (start 154.432 71.12) (end 154.432 72.644) (width 0.2) (layer "F.Cu") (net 2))
 (segment (start 146.05 70.612) (end 153.924 70.612) (width 0.2) (layer "F.Cu") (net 2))
 (segment (start 138.684 72.644) (end 138.684 71.12) (width 0.2) (layer "F.Cu") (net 2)))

